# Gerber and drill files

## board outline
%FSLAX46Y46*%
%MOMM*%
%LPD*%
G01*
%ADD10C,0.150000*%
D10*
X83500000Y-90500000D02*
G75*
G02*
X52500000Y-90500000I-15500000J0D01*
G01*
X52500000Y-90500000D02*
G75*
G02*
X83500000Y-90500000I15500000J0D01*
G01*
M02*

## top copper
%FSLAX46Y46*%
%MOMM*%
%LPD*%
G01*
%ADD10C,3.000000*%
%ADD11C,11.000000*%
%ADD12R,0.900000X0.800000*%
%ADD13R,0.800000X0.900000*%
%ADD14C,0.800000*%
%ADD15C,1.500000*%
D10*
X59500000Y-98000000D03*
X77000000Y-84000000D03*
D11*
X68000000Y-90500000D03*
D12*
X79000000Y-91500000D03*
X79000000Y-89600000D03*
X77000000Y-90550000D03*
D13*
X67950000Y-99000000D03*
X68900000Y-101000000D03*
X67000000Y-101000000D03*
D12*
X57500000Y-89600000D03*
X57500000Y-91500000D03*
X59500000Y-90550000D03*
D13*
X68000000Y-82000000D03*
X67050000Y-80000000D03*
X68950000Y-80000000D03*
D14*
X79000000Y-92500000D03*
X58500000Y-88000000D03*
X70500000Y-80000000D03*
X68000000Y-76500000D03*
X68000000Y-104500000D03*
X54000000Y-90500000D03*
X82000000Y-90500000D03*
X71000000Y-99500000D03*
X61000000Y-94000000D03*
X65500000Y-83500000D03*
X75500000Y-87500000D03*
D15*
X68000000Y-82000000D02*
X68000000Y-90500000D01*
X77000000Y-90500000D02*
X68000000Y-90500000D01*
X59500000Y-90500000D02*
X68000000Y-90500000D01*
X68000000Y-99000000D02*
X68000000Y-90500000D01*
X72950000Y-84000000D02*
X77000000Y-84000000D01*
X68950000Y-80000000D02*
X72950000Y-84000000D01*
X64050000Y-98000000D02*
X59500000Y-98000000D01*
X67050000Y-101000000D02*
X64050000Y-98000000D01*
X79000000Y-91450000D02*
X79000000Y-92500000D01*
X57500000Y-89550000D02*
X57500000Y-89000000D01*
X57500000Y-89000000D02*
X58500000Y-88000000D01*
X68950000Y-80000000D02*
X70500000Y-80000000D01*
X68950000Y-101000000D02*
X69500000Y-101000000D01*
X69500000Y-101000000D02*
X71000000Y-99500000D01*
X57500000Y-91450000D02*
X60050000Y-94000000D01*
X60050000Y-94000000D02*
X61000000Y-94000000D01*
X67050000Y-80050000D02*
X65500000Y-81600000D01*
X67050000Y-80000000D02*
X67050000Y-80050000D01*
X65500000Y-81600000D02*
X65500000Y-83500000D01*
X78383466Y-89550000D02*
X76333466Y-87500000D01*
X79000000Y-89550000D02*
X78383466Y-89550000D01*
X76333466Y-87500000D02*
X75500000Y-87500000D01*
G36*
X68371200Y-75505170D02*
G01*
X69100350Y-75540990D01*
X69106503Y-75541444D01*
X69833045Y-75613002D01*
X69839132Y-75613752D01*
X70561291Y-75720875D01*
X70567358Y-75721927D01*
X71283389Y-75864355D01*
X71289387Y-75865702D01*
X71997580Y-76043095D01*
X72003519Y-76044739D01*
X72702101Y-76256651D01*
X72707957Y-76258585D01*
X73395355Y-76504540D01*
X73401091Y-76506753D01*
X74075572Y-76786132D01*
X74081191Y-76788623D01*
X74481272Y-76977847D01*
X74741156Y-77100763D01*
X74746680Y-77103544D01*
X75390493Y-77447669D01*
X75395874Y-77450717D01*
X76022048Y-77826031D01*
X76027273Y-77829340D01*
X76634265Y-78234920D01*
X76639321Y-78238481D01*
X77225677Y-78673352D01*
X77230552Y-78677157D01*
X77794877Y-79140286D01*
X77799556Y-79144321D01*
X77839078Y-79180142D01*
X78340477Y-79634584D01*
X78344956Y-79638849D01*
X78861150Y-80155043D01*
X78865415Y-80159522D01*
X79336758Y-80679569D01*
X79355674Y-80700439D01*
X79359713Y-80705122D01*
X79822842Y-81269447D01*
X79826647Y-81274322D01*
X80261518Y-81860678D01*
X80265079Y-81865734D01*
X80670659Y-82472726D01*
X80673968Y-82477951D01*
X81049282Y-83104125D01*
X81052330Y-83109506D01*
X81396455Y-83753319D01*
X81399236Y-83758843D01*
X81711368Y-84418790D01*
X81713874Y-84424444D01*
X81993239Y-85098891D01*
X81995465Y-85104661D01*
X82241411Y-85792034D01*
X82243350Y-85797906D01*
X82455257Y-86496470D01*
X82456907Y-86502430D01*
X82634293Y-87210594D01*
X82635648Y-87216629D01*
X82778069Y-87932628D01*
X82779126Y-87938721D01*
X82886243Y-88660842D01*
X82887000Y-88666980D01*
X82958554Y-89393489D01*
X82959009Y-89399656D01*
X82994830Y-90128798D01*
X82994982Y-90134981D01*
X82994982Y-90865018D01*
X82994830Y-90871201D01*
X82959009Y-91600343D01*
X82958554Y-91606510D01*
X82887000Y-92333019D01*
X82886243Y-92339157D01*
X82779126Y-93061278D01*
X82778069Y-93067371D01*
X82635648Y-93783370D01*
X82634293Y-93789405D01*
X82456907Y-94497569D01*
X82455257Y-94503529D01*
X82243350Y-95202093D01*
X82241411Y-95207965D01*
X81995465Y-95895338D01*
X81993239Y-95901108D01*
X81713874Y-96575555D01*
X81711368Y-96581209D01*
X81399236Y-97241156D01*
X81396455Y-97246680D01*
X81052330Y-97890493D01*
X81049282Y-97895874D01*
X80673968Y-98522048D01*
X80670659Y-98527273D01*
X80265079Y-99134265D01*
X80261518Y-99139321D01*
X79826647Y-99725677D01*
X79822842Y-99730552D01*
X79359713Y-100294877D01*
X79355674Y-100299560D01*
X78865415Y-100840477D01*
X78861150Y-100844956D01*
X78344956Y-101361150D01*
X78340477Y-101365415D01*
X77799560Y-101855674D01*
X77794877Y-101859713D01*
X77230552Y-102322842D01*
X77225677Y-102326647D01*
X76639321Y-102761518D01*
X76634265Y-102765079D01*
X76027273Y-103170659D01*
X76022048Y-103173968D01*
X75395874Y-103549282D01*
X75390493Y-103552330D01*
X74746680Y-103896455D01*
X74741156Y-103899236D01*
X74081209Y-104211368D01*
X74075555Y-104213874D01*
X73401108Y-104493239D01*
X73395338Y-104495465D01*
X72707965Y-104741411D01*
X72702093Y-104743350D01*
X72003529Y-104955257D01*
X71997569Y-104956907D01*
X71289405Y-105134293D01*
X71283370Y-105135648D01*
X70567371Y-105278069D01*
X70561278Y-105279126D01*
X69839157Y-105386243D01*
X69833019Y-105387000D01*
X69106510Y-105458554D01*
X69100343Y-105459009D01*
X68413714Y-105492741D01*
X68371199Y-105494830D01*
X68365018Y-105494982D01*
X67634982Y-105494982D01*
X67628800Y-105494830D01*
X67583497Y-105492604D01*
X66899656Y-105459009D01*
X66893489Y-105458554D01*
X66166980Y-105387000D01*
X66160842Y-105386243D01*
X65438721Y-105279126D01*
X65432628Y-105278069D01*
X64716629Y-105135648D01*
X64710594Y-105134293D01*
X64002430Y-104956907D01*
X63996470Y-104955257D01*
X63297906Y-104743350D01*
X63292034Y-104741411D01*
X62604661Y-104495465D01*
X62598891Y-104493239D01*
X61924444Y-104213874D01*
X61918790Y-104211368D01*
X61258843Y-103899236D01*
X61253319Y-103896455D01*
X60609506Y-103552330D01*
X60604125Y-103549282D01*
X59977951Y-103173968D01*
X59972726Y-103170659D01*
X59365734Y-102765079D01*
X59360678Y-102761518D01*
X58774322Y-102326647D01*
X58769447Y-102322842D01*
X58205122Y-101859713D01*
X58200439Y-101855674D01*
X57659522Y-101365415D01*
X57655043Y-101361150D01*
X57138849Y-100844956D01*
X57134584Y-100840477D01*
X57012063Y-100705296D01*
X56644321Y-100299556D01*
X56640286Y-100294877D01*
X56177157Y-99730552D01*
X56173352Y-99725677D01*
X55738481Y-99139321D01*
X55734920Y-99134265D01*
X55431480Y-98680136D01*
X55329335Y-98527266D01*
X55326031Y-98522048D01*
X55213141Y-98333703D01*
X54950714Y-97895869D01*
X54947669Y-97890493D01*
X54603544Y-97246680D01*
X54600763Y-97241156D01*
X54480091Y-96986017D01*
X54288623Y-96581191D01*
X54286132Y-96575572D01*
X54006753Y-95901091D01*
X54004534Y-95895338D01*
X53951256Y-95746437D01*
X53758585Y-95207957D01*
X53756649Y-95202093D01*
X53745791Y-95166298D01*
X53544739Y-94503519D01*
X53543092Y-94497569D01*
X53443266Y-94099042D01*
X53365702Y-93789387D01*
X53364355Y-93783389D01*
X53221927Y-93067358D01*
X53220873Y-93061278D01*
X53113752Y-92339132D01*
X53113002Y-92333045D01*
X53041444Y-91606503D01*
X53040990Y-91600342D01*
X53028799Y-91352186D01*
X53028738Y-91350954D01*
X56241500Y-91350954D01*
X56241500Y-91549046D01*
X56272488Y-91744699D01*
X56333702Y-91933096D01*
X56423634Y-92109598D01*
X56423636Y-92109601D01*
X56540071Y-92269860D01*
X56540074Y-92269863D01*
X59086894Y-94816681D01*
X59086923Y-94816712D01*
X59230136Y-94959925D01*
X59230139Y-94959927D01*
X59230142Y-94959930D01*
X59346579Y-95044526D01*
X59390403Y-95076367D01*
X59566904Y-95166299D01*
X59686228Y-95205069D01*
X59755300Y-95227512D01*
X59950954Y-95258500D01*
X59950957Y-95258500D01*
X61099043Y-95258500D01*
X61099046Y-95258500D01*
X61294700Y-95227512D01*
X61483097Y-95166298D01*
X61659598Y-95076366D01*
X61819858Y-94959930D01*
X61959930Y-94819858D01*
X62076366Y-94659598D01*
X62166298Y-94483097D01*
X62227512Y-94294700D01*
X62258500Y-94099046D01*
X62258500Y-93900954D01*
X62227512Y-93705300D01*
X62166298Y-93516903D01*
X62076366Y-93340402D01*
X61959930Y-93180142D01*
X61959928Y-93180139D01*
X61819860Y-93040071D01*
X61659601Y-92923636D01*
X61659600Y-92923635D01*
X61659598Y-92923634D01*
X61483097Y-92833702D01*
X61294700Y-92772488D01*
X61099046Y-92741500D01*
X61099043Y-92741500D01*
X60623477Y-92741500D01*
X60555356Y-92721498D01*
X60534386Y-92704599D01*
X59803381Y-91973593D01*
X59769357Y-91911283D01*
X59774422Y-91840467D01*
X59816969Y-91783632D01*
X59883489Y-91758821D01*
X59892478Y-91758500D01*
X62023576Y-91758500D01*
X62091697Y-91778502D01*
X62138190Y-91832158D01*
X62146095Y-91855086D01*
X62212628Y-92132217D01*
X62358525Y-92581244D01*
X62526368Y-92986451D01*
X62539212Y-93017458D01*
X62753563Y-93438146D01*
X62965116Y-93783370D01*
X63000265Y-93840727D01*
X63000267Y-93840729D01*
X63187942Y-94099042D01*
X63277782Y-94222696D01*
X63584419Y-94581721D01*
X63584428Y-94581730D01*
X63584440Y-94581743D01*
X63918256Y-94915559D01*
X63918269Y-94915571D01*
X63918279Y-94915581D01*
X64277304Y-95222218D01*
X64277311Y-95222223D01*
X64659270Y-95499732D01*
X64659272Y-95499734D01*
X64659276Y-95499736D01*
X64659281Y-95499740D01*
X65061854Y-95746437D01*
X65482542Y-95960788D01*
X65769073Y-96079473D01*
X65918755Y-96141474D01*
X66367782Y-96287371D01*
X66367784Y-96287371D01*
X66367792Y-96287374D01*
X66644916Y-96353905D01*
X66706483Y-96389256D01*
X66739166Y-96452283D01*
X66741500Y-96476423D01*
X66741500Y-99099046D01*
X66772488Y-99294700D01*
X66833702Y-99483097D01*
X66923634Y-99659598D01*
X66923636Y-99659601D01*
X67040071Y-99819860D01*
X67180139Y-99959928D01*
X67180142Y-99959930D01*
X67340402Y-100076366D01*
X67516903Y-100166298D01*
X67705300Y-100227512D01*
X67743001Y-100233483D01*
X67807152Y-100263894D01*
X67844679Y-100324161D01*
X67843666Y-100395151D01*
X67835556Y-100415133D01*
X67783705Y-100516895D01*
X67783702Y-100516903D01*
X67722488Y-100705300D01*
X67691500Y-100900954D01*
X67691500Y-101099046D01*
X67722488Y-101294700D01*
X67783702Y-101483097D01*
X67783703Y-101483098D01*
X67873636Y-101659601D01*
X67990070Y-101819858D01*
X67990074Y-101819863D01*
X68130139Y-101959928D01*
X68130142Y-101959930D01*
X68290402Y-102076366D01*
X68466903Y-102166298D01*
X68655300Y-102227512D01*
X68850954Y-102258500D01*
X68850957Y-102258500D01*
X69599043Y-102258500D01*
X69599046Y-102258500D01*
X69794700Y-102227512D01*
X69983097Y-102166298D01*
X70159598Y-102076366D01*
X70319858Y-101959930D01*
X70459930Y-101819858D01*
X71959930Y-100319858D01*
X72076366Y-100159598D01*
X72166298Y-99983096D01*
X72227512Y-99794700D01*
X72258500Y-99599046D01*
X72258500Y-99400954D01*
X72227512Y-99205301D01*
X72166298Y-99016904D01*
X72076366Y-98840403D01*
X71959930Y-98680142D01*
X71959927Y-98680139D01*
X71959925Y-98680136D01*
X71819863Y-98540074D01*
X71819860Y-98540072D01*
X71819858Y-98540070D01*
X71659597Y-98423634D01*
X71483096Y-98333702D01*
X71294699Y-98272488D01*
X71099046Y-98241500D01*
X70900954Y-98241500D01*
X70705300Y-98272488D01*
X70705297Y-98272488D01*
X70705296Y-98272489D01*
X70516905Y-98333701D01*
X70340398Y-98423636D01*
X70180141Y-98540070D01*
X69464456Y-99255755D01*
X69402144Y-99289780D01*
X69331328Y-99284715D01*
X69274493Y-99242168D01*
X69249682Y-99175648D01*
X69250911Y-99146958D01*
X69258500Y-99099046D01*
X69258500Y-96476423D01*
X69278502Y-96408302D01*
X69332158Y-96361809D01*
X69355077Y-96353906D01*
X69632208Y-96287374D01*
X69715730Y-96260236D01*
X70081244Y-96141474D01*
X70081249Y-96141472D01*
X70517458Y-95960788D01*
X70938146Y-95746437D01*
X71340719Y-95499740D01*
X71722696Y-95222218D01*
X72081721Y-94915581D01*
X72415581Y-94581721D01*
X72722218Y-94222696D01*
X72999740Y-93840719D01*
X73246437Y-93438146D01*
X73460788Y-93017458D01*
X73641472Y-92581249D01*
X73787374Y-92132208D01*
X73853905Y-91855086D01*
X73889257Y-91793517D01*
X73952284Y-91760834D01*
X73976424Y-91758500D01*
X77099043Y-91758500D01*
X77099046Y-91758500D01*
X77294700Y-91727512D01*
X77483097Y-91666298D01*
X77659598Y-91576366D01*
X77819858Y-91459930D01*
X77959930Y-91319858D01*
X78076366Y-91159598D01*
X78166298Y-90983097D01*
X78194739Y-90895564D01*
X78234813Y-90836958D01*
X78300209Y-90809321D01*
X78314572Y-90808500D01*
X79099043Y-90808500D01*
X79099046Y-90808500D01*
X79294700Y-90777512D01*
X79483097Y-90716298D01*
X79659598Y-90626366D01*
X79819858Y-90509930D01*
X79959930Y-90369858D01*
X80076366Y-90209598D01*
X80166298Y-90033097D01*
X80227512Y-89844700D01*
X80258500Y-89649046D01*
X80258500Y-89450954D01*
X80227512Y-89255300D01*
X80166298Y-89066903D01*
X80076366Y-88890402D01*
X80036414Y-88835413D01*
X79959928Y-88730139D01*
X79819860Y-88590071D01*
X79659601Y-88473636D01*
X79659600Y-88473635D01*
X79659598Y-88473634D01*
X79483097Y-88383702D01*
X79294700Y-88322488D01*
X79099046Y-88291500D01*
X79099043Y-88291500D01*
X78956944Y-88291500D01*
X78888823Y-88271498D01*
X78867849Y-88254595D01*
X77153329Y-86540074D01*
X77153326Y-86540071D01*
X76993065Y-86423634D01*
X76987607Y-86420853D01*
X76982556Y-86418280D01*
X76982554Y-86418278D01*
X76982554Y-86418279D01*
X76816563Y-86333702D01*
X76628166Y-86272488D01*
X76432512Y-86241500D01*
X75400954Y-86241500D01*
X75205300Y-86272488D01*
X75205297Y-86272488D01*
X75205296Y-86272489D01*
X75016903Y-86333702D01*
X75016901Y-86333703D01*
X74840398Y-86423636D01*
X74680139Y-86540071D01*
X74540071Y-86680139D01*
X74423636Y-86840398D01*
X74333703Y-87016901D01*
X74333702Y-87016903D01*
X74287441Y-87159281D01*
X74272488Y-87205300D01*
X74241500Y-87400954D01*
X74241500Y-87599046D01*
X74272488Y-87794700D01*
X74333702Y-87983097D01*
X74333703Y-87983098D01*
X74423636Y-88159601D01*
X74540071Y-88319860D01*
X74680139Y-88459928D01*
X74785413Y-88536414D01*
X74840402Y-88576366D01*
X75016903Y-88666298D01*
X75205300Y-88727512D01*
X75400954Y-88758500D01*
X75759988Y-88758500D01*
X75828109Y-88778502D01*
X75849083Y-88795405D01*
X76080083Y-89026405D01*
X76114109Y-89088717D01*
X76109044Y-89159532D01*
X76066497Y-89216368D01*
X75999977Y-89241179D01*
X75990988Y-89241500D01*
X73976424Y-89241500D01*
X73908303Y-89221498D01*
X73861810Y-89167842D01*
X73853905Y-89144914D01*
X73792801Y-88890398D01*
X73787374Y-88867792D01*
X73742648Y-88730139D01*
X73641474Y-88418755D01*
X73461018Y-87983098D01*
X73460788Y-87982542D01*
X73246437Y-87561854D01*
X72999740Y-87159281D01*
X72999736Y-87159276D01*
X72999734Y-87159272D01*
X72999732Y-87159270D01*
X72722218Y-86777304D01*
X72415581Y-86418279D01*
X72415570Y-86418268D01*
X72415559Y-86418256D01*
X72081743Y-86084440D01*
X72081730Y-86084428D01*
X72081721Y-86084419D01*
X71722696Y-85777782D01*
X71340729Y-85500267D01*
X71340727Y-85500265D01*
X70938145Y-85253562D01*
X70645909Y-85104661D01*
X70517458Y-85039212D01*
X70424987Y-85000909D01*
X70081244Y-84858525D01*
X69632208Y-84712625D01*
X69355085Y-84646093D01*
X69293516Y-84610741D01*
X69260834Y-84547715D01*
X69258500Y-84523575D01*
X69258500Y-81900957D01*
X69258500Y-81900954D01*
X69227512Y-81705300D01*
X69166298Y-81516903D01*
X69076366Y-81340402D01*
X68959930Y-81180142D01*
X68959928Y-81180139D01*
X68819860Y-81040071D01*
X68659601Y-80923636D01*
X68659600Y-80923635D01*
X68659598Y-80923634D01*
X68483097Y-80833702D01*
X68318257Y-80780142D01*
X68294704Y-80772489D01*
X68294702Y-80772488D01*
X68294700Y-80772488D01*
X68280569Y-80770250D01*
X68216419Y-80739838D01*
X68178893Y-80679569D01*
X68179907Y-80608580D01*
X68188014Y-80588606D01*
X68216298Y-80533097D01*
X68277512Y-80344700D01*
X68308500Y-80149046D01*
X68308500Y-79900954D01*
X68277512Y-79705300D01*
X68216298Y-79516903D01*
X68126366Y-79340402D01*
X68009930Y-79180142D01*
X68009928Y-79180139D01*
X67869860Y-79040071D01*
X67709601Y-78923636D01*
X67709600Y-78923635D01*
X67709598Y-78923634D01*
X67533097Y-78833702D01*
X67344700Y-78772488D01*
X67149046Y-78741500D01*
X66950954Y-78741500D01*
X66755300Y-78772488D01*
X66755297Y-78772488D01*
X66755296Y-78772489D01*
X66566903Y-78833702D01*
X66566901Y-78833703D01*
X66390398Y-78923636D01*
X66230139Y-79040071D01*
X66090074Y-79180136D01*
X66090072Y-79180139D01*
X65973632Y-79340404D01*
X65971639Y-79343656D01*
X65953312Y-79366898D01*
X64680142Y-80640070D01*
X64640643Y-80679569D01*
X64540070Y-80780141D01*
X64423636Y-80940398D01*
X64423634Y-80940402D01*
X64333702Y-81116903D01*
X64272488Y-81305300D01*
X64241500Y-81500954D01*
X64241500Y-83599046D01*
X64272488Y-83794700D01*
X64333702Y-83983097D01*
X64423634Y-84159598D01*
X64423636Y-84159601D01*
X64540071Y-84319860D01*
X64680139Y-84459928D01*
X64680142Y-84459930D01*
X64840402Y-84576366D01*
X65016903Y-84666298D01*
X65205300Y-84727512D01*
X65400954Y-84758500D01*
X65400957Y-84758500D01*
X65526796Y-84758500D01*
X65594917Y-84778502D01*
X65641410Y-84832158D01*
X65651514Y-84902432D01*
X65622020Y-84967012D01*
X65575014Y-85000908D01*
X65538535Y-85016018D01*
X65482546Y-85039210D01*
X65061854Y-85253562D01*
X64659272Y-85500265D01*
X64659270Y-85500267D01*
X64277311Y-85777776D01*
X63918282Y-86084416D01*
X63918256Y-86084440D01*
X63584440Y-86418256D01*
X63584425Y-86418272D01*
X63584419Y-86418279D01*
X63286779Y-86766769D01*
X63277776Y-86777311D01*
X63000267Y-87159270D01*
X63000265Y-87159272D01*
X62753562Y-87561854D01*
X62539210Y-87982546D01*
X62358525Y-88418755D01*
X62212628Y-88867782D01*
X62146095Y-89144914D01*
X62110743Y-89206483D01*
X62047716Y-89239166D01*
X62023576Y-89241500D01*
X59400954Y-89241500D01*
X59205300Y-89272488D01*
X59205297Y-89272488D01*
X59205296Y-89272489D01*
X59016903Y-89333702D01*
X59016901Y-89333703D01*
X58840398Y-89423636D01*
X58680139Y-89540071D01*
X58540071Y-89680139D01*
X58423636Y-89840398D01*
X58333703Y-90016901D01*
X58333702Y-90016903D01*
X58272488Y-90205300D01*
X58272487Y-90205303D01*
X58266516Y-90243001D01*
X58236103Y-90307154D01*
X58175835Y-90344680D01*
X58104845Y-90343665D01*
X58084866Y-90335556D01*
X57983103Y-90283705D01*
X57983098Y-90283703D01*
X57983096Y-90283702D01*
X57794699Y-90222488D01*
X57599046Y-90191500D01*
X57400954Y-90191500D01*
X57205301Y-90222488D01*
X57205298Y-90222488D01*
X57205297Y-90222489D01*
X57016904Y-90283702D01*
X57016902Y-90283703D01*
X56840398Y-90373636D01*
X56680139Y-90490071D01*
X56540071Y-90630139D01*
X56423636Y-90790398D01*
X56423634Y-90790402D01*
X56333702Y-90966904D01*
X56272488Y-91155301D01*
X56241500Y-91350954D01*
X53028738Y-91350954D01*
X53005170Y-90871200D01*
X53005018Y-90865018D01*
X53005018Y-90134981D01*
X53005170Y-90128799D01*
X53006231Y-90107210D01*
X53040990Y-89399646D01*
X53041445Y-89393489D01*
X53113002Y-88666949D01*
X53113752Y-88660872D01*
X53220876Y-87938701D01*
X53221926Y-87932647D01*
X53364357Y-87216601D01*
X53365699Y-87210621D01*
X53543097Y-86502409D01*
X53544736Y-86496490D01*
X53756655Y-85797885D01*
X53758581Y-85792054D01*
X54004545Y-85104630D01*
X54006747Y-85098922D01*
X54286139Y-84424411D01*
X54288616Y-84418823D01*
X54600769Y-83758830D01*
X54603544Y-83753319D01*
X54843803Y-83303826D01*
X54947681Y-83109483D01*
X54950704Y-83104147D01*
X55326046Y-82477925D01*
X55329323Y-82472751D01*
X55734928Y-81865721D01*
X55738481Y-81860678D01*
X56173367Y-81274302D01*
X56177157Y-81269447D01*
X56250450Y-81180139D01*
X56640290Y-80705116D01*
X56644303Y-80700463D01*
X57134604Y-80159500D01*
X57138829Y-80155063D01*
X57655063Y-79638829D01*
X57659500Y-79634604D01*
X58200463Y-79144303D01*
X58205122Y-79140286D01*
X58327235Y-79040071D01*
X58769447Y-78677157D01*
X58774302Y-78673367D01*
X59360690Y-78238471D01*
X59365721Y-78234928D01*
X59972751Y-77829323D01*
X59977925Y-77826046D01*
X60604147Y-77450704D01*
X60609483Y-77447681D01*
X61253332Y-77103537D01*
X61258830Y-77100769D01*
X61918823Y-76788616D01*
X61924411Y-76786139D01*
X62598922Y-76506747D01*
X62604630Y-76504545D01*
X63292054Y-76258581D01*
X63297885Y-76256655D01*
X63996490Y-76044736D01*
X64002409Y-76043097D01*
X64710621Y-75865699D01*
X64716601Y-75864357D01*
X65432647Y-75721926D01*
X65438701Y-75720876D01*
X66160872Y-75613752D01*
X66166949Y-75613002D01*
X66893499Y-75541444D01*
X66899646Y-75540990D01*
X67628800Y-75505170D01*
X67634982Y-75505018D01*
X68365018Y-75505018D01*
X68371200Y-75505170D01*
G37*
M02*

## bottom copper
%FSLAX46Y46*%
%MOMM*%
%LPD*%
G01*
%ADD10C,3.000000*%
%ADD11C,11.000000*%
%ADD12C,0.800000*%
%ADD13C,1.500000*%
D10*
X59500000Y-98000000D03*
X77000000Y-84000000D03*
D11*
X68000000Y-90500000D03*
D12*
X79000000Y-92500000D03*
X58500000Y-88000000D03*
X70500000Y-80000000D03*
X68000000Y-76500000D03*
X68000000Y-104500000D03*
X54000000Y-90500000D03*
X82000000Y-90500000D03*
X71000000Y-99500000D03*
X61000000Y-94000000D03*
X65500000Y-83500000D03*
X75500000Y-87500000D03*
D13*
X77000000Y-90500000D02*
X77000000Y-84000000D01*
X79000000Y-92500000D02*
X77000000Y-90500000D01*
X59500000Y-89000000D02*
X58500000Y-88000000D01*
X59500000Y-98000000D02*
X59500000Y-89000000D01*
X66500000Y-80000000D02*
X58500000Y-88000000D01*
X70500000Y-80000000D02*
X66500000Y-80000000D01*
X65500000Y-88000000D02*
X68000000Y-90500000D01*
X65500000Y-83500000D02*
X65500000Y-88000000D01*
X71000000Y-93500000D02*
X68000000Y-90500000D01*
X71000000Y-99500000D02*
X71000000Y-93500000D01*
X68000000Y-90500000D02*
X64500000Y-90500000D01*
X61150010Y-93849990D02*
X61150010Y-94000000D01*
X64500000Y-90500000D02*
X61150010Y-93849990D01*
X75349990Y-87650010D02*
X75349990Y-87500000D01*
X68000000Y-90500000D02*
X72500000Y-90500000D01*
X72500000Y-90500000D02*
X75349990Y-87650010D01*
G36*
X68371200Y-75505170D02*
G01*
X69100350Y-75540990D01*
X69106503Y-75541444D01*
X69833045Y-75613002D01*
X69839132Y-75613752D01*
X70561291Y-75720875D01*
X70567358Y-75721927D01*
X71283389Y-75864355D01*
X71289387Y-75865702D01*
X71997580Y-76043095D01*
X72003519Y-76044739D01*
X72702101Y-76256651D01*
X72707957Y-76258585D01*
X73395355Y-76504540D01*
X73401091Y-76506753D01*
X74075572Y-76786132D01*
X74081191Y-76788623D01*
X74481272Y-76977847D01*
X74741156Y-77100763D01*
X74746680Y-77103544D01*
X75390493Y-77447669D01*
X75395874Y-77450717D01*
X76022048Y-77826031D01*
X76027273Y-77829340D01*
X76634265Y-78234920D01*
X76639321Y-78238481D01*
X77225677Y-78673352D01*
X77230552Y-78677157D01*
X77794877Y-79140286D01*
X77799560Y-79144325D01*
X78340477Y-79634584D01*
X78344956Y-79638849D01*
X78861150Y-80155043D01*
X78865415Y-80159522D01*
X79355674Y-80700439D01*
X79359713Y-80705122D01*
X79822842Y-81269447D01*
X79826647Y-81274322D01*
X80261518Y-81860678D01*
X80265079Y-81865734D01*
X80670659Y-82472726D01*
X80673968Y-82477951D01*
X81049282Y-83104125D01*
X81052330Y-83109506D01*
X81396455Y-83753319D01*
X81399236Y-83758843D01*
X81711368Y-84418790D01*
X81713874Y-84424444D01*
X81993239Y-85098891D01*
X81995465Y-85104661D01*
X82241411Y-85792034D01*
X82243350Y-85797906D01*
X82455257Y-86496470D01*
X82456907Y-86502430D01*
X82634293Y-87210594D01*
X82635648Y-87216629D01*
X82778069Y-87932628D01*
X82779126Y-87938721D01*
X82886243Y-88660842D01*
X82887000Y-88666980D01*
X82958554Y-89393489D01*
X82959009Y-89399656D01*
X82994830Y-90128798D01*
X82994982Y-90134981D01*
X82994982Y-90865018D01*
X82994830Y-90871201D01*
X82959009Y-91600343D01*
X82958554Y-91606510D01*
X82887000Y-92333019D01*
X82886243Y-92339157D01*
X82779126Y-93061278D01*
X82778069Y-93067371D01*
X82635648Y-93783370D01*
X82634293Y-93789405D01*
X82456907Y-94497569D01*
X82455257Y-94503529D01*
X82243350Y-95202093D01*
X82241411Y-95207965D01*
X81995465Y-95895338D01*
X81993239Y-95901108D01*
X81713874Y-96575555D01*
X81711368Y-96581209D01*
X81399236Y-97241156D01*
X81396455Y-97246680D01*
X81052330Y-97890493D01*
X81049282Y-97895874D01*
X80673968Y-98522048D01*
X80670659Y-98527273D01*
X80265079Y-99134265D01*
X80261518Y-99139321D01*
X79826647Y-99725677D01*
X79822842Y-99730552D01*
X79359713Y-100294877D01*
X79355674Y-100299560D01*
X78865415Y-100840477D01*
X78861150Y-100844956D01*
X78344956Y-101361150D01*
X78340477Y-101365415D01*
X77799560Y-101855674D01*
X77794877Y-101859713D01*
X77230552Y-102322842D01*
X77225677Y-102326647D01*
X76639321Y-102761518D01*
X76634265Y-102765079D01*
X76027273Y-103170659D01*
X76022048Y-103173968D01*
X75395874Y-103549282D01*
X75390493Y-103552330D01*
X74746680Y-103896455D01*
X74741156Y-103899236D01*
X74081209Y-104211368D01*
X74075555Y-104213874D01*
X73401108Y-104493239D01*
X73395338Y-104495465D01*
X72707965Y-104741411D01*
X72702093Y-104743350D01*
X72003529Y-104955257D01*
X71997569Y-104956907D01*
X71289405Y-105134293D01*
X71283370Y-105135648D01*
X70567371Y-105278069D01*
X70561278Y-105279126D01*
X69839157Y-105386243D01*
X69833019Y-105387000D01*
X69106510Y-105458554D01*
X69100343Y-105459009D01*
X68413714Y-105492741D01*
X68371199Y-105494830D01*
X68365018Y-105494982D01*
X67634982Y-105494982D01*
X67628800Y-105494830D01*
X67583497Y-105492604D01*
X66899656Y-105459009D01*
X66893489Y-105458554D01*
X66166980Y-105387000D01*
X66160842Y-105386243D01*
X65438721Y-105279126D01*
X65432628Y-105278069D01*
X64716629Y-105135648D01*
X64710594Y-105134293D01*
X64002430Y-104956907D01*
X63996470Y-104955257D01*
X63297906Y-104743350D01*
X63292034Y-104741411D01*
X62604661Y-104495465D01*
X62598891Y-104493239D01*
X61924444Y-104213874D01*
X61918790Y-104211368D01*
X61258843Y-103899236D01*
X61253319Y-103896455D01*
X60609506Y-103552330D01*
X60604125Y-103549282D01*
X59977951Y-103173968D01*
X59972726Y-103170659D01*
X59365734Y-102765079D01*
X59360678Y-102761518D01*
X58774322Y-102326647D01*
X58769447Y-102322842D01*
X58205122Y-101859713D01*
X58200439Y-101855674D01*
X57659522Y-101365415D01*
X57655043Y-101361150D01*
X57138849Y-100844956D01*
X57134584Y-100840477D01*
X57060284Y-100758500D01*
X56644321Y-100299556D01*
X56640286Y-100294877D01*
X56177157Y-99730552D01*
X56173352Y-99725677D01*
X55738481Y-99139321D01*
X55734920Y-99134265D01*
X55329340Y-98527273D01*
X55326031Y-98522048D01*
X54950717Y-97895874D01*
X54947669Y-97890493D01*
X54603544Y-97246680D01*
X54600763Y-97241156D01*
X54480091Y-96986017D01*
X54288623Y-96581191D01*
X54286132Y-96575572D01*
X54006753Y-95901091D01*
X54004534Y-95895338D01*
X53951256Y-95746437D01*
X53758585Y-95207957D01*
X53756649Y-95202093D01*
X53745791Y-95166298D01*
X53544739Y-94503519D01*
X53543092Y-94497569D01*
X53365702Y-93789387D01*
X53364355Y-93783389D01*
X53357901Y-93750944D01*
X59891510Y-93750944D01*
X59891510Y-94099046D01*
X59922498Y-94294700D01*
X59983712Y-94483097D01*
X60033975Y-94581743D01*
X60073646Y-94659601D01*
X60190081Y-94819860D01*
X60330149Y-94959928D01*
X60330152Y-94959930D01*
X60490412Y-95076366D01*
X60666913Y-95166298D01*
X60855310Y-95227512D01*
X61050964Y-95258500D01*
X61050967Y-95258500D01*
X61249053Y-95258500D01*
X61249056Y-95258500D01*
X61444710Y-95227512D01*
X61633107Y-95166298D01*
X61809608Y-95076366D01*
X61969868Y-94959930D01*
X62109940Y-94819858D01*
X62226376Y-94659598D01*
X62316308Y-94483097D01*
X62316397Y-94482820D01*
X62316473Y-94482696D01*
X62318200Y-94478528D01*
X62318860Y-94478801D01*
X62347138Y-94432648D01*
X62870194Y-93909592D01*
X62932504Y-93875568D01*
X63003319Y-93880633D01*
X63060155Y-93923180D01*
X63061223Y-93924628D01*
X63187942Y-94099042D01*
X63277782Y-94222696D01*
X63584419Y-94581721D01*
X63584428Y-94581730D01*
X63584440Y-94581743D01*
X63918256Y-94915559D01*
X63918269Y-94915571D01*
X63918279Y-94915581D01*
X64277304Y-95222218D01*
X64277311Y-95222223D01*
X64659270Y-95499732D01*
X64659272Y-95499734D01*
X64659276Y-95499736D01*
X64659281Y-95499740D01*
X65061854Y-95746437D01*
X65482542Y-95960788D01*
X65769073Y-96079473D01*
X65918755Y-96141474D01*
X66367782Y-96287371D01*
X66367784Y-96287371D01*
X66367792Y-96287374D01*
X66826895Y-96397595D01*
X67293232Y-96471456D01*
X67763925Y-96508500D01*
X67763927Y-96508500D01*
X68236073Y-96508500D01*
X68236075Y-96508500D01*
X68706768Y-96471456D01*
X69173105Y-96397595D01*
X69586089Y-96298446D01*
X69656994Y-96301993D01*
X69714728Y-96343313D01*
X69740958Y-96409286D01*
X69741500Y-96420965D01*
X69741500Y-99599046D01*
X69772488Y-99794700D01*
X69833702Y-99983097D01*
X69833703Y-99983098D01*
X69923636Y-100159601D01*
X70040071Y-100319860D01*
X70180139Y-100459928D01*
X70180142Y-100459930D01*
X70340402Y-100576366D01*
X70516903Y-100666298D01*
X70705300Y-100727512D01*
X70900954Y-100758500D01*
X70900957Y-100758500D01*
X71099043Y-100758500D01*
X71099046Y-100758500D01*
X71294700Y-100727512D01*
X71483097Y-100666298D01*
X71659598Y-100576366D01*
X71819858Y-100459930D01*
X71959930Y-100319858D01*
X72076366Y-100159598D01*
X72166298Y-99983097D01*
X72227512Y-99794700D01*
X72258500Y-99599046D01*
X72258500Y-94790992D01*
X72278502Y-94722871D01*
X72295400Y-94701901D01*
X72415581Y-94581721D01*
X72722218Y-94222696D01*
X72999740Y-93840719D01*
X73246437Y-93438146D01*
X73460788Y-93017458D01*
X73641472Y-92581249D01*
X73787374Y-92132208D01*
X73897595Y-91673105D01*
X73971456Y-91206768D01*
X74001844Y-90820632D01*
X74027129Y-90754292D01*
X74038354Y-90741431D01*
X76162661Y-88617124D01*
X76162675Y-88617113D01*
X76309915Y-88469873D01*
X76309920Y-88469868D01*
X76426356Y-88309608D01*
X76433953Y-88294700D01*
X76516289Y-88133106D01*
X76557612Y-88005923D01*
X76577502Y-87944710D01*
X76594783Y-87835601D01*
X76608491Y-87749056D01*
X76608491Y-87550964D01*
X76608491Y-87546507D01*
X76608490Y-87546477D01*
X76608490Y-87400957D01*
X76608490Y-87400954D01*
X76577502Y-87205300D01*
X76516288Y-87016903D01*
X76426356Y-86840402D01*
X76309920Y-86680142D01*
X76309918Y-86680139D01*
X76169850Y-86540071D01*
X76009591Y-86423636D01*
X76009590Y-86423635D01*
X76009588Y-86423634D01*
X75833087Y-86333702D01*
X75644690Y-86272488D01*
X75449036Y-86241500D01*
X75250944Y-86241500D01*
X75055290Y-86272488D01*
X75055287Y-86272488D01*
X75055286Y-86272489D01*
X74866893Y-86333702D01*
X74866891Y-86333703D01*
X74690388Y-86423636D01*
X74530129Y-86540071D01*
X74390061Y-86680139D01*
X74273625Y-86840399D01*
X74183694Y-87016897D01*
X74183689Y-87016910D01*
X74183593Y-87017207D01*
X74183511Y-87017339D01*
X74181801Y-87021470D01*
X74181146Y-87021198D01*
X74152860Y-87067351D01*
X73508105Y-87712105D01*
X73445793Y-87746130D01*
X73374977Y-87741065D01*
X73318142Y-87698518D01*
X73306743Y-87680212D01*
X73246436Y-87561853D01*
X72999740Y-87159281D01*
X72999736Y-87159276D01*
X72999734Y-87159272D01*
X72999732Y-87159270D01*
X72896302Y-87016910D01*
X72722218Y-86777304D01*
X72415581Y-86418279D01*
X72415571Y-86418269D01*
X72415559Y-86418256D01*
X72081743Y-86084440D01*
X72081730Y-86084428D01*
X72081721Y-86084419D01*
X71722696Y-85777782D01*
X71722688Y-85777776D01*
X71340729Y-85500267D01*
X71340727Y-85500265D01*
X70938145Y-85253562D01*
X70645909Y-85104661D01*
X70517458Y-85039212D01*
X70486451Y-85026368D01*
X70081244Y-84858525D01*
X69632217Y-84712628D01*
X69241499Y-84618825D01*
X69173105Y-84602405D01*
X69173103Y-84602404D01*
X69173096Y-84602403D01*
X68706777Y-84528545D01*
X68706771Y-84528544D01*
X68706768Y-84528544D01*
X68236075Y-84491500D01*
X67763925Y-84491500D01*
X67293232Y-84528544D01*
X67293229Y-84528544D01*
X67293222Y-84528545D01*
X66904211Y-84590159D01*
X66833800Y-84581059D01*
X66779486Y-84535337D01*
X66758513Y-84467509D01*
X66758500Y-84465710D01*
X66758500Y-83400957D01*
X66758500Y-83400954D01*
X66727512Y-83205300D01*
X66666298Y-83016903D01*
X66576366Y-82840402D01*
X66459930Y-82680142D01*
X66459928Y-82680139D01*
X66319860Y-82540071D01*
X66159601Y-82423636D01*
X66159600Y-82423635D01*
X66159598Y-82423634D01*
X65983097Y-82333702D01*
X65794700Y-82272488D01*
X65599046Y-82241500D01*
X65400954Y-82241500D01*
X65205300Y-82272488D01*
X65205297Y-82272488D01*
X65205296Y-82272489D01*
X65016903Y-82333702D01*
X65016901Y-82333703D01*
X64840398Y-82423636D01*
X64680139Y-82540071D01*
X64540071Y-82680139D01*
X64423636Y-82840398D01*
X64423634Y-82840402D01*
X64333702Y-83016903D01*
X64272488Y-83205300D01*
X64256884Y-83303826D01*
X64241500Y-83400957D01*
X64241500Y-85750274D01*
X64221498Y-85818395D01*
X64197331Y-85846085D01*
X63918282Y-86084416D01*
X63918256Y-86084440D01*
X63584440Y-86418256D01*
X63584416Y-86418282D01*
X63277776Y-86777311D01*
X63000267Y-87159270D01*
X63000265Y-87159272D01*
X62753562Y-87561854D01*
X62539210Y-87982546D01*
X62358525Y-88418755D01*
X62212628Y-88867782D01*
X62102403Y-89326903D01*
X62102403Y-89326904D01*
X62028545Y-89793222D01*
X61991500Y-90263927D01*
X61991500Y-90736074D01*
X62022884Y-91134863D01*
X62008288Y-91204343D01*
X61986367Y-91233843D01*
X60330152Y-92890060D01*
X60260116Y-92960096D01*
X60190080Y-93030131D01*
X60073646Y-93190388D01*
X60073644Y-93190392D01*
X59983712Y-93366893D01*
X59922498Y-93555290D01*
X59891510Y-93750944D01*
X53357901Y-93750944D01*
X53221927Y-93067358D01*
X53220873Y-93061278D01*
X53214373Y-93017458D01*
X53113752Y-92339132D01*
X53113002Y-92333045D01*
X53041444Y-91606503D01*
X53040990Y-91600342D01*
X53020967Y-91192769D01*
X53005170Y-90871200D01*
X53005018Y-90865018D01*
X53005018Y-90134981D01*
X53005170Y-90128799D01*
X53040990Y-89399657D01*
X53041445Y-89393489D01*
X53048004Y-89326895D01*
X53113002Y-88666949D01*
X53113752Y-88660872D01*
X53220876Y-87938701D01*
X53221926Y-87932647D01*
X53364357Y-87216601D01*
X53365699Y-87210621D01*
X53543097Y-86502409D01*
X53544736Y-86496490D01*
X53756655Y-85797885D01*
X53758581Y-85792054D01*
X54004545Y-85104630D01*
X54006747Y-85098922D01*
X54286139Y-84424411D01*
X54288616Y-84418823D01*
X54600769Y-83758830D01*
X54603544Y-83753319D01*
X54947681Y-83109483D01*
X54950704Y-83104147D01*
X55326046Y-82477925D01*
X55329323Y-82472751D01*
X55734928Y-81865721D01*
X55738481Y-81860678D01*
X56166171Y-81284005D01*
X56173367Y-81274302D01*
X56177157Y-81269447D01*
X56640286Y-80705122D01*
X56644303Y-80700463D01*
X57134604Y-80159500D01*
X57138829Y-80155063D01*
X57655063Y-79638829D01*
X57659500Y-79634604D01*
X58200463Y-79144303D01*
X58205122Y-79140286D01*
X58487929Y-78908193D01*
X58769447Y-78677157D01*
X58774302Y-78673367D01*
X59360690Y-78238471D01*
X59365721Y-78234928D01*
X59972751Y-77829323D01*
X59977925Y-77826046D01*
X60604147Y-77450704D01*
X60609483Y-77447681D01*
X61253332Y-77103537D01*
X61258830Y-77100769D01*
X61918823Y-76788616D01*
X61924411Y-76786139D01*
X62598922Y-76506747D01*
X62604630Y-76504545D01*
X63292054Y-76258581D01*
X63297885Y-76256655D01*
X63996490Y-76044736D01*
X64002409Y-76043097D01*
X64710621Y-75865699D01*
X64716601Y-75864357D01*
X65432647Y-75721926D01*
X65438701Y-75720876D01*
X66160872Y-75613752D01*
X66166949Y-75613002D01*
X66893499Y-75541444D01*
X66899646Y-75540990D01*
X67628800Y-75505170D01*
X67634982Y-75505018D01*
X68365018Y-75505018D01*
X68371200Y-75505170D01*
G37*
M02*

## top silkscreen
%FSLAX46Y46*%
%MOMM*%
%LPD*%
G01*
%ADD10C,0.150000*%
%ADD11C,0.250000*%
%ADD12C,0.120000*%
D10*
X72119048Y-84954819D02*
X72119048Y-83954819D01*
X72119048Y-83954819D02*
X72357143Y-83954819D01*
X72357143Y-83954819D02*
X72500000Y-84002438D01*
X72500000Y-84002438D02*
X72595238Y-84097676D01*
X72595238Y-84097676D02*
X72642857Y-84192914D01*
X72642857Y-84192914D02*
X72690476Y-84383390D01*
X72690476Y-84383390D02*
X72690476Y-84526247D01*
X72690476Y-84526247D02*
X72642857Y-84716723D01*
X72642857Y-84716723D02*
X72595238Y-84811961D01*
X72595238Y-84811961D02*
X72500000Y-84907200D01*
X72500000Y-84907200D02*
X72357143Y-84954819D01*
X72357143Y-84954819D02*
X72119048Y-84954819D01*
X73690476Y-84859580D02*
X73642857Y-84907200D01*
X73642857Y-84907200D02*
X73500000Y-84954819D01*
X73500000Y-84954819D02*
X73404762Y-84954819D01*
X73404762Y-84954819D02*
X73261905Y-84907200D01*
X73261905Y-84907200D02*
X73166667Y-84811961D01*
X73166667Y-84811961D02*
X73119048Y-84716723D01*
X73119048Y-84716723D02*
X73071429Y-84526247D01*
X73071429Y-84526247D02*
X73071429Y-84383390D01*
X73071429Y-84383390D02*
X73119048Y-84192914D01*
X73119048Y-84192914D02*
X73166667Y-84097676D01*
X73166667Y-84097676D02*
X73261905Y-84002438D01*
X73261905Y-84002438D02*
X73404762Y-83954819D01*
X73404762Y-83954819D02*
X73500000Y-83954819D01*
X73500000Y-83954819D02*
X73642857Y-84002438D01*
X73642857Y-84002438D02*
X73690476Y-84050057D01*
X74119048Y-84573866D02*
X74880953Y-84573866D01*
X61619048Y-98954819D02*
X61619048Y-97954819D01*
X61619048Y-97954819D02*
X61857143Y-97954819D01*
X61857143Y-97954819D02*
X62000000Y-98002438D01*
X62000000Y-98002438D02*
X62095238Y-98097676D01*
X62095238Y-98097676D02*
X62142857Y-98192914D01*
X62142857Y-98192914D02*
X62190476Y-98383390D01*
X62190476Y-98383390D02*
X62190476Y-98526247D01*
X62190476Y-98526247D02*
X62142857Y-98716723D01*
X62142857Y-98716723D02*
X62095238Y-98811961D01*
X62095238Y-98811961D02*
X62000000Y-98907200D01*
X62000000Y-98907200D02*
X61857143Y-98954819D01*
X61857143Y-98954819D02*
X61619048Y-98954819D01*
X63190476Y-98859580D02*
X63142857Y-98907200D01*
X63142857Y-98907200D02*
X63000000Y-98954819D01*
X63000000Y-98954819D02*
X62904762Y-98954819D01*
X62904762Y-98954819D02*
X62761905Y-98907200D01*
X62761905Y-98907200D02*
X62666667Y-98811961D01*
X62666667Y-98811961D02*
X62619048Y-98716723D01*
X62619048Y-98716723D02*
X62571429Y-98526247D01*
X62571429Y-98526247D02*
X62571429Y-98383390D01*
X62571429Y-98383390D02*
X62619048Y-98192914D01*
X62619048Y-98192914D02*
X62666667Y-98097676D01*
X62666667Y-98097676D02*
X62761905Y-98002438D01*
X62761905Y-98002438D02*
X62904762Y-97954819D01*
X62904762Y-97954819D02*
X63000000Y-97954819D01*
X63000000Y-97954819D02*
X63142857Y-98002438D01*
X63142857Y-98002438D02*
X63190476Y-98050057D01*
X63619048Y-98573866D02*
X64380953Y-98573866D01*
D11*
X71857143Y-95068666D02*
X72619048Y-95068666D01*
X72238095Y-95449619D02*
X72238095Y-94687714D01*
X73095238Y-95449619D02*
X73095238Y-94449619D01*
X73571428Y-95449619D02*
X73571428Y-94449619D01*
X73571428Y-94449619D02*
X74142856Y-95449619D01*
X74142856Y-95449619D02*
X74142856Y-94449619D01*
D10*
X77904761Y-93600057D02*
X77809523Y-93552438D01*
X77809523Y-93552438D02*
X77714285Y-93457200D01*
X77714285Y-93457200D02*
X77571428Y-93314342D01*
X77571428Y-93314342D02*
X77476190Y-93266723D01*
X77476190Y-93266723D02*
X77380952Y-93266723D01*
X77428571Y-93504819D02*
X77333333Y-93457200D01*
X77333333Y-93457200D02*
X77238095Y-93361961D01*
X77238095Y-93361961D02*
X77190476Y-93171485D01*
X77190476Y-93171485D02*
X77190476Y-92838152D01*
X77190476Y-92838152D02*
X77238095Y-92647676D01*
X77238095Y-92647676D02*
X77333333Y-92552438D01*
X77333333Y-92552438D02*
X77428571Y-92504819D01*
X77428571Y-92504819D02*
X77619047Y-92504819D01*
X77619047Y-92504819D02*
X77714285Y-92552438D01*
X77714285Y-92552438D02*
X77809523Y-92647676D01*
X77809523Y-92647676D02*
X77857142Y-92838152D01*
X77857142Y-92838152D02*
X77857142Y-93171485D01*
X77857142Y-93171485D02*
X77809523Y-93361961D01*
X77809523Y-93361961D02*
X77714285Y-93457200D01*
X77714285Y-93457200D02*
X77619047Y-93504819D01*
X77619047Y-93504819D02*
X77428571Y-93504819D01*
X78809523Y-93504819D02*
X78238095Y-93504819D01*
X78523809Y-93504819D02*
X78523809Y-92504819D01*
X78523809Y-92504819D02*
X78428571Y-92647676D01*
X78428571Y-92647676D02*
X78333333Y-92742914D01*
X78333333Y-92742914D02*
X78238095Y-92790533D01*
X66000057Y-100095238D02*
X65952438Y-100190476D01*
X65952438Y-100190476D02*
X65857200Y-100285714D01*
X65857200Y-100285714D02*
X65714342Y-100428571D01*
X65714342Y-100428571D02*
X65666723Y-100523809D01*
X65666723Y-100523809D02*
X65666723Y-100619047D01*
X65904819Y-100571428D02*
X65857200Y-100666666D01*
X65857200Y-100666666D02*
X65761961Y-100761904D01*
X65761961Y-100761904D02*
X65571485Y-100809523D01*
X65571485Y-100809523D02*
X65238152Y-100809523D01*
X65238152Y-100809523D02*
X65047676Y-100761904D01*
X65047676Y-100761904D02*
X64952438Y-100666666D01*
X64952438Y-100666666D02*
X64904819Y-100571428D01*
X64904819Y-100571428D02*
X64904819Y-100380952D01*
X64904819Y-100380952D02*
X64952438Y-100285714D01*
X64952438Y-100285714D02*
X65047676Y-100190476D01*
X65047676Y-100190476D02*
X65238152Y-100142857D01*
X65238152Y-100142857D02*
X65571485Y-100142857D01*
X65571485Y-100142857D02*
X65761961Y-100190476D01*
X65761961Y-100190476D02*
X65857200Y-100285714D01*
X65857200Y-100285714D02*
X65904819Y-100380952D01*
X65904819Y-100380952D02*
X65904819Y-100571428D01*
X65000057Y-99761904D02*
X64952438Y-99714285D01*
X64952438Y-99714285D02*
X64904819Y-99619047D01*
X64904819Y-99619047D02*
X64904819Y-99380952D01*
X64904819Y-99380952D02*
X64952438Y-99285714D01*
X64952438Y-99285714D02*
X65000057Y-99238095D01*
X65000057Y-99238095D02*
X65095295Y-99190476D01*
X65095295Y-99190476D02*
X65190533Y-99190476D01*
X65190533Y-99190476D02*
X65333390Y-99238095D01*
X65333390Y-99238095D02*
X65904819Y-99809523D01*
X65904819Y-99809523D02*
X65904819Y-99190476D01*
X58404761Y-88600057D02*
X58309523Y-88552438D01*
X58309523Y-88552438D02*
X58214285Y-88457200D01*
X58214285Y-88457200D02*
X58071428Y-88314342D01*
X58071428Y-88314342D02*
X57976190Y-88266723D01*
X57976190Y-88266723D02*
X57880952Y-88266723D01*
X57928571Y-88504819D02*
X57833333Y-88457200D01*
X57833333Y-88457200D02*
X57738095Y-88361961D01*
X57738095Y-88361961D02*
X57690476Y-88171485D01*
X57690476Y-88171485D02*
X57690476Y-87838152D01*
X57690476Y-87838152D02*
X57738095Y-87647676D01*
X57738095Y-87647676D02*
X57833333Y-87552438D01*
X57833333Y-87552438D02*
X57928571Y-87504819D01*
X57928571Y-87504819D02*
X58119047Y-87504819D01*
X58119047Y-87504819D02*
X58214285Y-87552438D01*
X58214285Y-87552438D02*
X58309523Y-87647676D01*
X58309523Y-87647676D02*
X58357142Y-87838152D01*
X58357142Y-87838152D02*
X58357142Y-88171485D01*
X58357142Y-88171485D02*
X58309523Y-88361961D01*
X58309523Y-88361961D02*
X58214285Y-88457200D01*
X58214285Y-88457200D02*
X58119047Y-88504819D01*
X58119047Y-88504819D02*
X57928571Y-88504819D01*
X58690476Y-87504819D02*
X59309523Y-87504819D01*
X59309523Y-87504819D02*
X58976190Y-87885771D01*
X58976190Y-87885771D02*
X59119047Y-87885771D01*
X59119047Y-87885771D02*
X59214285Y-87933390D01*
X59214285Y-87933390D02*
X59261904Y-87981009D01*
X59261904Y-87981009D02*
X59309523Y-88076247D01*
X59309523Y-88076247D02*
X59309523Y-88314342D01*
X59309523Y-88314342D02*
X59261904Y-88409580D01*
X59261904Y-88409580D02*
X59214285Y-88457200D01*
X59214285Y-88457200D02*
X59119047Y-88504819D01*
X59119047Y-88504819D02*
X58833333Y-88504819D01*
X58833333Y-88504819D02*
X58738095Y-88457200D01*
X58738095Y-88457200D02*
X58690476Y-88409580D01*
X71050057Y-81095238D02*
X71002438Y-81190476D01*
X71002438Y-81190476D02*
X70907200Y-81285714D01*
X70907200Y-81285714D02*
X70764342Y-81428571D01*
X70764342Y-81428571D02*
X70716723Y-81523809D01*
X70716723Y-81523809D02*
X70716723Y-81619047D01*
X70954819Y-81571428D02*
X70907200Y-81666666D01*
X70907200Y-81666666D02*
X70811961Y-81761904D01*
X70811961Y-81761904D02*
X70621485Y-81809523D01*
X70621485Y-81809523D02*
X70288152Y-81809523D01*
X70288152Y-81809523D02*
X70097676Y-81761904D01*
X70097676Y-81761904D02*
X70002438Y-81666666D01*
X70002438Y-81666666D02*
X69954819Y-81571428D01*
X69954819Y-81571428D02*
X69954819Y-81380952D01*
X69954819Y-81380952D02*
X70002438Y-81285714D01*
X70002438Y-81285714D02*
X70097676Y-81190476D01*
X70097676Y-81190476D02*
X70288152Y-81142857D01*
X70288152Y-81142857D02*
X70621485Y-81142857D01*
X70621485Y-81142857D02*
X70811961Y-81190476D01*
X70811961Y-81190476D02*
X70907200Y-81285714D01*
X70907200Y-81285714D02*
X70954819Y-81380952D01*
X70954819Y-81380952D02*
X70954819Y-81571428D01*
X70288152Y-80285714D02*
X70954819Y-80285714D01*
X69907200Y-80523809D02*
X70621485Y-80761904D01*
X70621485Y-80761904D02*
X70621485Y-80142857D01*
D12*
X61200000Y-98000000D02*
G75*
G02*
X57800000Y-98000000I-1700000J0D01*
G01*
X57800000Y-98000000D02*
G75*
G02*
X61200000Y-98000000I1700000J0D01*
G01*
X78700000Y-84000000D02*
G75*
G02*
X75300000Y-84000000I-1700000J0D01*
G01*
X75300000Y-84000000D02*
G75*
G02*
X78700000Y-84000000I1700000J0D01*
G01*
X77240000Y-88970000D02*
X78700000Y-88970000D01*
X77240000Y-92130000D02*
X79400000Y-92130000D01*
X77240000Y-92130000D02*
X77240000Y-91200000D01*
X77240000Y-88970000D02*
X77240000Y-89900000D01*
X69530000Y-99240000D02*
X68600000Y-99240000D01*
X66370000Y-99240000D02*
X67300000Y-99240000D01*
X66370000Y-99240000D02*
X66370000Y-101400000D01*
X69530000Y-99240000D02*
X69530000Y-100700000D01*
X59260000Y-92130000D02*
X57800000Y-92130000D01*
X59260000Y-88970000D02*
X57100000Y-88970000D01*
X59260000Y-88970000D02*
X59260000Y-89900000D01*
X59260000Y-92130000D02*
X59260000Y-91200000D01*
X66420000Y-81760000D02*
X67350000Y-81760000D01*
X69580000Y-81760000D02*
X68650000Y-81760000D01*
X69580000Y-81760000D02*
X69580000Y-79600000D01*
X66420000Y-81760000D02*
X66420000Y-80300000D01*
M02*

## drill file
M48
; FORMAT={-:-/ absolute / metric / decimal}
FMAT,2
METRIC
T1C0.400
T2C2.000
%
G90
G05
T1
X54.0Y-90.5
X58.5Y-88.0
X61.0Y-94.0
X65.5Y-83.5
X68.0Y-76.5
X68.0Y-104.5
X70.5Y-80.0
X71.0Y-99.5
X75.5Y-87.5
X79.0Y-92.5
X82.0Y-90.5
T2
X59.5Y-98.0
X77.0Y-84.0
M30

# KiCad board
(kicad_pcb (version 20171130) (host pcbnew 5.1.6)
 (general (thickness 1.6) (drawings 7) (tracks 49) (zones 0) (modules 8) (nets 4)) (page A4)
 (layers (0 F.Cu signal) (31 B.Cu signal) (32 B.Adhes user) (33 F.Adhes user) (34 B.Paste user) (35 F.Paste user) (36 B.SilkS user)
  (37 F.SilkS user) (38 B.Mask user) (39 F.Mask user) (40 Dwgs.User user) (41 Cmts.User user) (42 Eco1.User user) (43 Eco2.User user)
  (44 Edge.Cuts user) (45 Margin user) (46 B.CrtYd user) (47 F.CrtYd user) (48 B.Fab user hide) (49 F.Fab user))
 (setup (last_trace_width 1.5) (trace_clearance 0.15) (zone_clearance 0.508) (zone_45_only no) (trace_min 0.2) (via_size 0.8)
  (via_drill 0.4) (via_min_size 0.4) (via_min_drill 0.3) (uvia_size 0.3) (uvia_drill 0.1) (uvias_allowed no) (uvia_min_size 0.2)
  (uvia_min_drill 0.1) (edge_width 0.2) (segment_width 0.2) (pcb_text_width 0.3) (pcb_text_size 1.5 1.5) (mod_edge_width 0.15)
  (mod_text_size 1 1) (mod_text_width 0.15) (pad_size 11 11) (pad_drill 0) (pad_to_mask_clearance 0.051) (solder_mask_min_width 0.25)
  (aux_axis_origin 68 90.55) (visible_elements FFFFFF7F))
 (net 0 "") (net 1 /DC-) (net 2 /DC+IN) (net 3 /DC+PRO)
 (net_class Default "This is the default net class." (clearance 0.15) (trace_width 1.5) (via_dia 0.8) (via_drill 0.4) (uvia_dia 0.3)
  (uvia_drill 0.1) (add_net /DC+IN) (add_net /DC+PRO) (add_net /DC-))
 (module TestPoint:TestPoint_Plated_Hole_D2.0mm (layer F.Cu) (at 59.5 98)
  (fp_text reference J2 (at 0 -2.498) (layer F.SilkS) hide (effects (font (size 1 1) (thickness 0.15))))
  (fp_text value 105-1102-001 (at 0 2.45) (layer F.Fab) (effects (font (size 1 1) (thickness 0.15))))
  (fp_circle (center 0 0) (end 0 -1.7) (layer F.SilkS) (width 0.12))
  (pad 1 thru_hole circle (at 0 0) (size 3 3) (drill 2) (layers *.Cu *.Mask) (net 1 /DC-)))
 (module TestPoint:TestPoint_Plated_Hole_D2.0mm (layer F.Cu) (at 77 84)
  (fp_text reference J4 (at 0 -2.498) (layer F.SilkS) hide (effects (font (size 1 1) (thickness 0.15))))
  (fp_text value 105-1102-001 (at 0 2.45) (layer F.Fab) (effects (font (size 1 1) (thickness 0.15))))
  (fp_circle (center 0 0) (end 0 -1.7) (layer F.SilkS) (width 0.12))
  (pad 1 thru_hole circle (at 0 0) (size 3 3) (drill 2) (layers *.Cu *.Mask) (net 1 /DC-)))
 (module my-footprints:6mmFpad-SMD (layer F.Cu) (at 68 90.5)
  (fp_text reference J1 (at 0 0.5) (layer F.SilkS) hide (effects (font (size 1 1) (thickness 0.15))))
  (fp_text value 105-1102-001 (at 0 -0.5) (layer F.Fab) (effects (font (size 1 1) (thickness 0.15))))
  (pad 1 smd circle (at 0 0) (size 11 11) (layers F.Cu F.Paste F.Mask) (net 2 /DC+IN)))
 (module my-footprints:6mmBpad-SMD (layer F.Cu) (at 68 90.5)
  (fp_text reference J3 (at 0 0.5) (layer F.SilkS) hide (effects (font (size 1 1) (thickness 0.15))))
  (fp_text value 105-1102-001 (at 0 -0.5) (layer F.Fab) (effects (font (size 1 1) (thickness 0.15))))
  (pad 1 smd circle (at 0 0) (size 11 11) (layers B.Cu B.Paste B.Mask) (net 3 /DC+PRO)))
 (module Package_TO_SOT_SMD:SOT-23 (layer F.Cu) (at 78 90.55 180)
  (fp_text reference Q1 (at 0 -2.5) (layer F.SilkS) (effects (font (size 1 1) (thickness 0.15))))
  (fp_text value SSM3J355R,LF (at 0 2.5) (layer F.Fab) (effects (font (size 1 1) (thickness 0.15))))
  (fp_line (start 0.76 1.58) (end -0.7 1.58) (layer F.SilkS) (width 0.12))
  (fp_line (start 0.76 -1.58) (end -1.4 -1.58) (layer F.SilkS) (width 0.12))
  (fp_line (start 0.76 -1.58) (end 0.76 -0.65) (layer F.SilkS) (width 0.12))
  (fp_line (start 0.76 1.58) (end 0.76 0.65) (layer F.SilkS) (width 0.12))
  (pad 1 smd rect (at -1 -0.95 180) (size 0.9 0.8) (layers F.Cu F.Paste F.Mask) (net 1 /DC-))
  (pad 2 smd rect (at -1 0.95 180) (size 0.9 0.8) (layers F.Cu F.Paste F.Mask) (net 3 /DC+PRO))
  (pad 3 smd rect (at 1 0 180) (size 0.9 0.8) (layers F.Cu F.Paste F.Mask) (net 2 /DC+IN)))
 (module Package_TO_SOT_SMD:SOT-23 (layer F.Cu) (at 67.95 100 90)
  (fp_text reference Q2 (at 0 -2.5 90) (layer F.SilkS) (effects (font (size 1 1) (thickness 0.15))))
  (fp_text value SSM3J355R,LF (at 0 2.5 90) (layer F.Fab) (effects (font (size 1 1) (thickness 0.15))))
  (fp_line (start 0.76 1.58) (end 0.76 0.65) (layer F.SilkS) (width 0.12))
  (fp_line (start 0.76 -1.58) (end 0.76 -0.65) (layer F.SilkS) (width 0.12))
  (fp_line (start 0.76 -1.58) (end -1.4 -1.58) (layer F.SilkS) (width 0.12))
  (fp_line (start 0.76 1.58) (end -0.7 1.58) (layer F.SilkS) (width 0.12))
  (pad 3 smd rect (at 1 0 90) (size 0.9 0.8) (layers F.Cu F.Paste F.Mask) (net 2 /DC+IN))
  (pad 2 smd rect (at -1 0.95 90) (size 0.9 0.8) (layers F.Cu F.Paste F.Mask) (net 3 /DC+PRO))
  (pad 1 smd rect (at -1 -0.95 90) (size 0.9 0.8) (layers F.Cu F.Paste F.Mask) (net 1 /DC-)))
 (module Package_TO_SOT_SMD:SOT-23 (layer F.Cu) (at 58.5 90.55)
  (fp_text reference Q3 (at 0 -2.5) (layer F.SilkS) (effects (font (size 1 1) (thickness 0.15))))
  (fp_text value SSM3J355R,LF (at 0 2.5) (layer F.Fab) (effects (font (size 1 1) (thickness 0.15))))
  (fp_line (start 0.76 1.58) (end -0.7 1.58) (layer F.SilkS) (width 0.12))
  (fp_line (start 0.76 -1.58) (end -1.4 -1.58) (layer F.SilkS) (width 0.12))
  (fp_line (start 0.76 -1.58) (end 0.76 -0.65) (layer F.SilkS) (width 0.12))
  (fp_line (start 0.76 1.58) (end 0.76 0.65) (layer F.SilkS) (width 0.12))
  (pad 1 smd rect (at -1 -0.95) (size 0.9 0.8) (layers F.Cu F.Paste F.Mask) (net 1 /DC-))
  (pad 2 smd rect (at -1 0.95) (size 0.9 0.8) (layers F.Cu F.Paste F.Mask) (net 3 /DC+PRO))
  (pad 3 smd rect (at 1 0) (size 0.9 0.8) (layers F.Cu F.Paste F.Mask) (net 2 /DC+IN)))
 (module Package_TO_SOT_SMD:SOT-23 (layer F.Cu) (at 68 81 270)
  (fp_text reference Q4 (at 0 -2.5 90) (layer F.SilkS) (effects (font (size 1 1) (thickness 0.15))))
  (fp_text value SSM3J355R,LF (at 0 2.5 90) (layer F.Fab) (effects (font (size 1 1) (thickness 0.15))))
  (fp_line (start 0.76 1.58) (end 0.76 0.65) (layer F.SilkS) (width 0.12))
  (fp_line (start 0.76 -1.58) (end 0.76 -0.65) (layer F.SilkS) (width 0.12))
  (fp_line (start 0.76 -1.58) (end -1.4 -1.58) (layer F.SilkS) (width 0.12))
  (fp_line (start 0.76 1.58) (end -0.7 1.58) (layer F.SilkS) (width 0.12))
  (pad 3 smd rect (at 1 0 270) (size 0.9 0.8) (layers F.Cu F.Paste F.Mask) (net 2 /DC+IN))
  (pad 2 smd rect (at -1 0.95 270) (size 0.9 0.8) (layers F.Cu F.Paste F.Mask) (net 3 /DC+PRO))
  (pad 1 smd rect (at -1 -0.95 270) (size 0.9 0.8) (layers F.Cu F.Paste F.Mask) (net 1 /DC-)))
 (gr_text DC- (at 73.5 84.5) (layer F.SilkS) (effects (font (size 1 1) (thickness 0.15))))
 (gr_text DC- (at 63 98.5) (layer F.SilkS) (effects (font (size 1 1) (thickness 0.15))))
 (gr_circle (center 68 90.5) (end 83.5 90.5) (layer Edge.Cuts) (width 0.15))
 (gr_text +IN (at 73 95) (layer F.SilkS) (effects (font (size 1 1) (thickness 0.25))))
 (segment (start 68 82) (end 68 90.5) (width 1.5) (layer F.Cu) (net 2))
 (segment (start 77 90.5) (end 68 90.5) (width 1.5) (layer F.Cu) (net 2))
 (segment (start 59.5 90.5) (end 68 90.5) (width 1.5) (layer F.Cu) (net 2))
 (segment (start 68 99) (end 68 90.5) (width 1.5) (layer F.Cu) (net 2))
 (segment (start 72.95 84) (end 77 84) (width 1.5) (layer F.Cu) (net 1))
 (segment (start 68.95 80) (end 72.95 84) (width 1.5) (layer F.Cu) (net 1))
 (segment (start 64.05 98) (end 59.5 98) (width 1.5) (layer F.Cu) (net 1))
 (segment (start 67.05 101) (end 64.05 98) (width 1.5) (layer F.Cu) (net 1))
 (segment (start 79 91.45) (end 79 92.5) (width 1.5) (layer F.Cu) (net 1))
 (via (at 79 92.5) (size 0.8) (drill 0.4) (layers F.Cu B.Cu) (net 1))
 (segment (start 77 90.5) (end 77 84) (width 1.5) (layer B.Cu) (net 1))
 (segment (start 79 92.5) (end 77 90.5) (width 1.5) (layer B.Cu) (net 1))
 (segment (start 57.5 89.55) (end 57.5 89) (width 1.5) (layer F.Cu) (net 1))
 (via (at 58.5 88) (size 0.8) (drill 0.4) (layers F.Cu B.Cu) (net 1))
 (segment (start 57.5 89) (end 58.5 88) (width 1.5) (layer F.Cu) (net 1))
 (segment (start 59.5 89) (end 58.5 88) (width 1.5) (layer B.Cu) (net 1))
 (segment (start 59.5 98) (end 59.5 89) (width 1.5) (layer B.Cu) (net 1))
 (segment (start 68.95 80) (end 70.5 80) (width 1.5) (layer F.Cu) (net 1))
 (via (at 70.5 80) (size 0.8) (drill 0.4) (layers F.Cu B.Cu) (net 1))
 (segment (start 66.5 80) (end 58.5 88) (width 1.5) (layer B.Cu) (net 1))
 (segment (start 70.5 80) (end 66.5 80) (width 1.5) (layer B.Cu) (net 1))
 (via (at 68 76.5) (size 0.8) (drill 0.4) (layers F.Cu B.Cu) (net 1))
 (via (at 68 104.5) (size 0.8) (drill 0.4) (layers F.Cu B.Cu) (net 1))
 (via (at 54 90.5) (size 0.8) (drill 0.4) (layers F.Cu B.Cu) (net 1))
 (via (at 82 90.5) (size 0.8) (drill 0.4) (layers F.Cu B.Cu) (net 1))
 (via (at 71 99.5) (size 0.8) (drill 0.4) (layers F.Cu B.Cu) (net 3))
 (segment (start 68.95 101) (end 69.5 101) (width 1.5) (layer F.Cu) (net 3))
 (segment (start 69.5 101) (end 71 99.5) (width 1.5) (layer F.Cu) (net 3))
 (segment (start 57.5 91.45) (end 60.05 94) (width 1.5) (layer F.Cu) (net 3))
 (via (at 61 94) (size 0.8) (drill 0.4) (layers F.Cu B.Cu) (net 3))
 (segment (start 60.05 94) (end 61 94) (width 1.5) (layer F.Cu) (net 3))
 (segment (start 67.05 80.05) (end 65.5 81.6) (width 1.5) (layer F.Cu) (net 3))
 (segment (start 67.05 80) (end 67.05 80.05) (width 1.5) (layer F.Cu) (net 3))
 (via (at 65.5 83.5) (size 0.8) (drill 0.4) (layers F.Cu B.Cu) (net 3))
 (segment (start 65.5 81.6) (end 65.5 83.5) (width 1.5) (layer F.Cu) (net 3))
 (segment (start 65.5 88) (end 68 90.5) (width 1.5) (layer B.Cu) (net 3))
 (segment (start 65.5 83.5) (end 65.5 88) (width 1.5) (layer B.Cu) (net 3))
 (segment (start 71 93.5) (end 68 90.5) (width 1.5) (layer B.Cu) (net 3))
 (segment (start 71 99.5) (end 71 93.5) (width 1.5) (layer B.Cu) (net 3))
 (segment (start 68 90.5) (end 64.5 90.5) (width 1.5) (layer B.Cu) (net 3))
 (segment (start 61.15001 93.84999) (end 61.15001 94) (width 1.5) (layer B.Cu) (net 3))
 (segment (start 64.5 90.5) (end 61.15001 93.84999) (width 1.5) (layer B.Cu) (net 3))
 (segment (start 78.383466 89.55) (end 76.333466 87.5) (width 1.5) (layer F.Cu) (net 3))
 (segment (start 79 89.55) (end 78.383466 89.55) (width 1.5) (layer F.Cu) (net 3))
 (via (at 75.5 87.5) (size 0.8) (drill 0.4) (layers F.Cu B.Cu) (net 3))
 (segment (start 76.333466 87.5) (end 75.5 87.5) (width 1.5) (layer F.Cu) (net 3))
 (segment (start 75.34999 87.65001) (end 75.34999 87.5) (width 1.5) (layer B.Cu) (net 3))
 (segment (start 68 90.5) (end 72.5 90.5) (width 1.5) (layer B.Cu) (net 3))
 (segment (start 72.5 90.5) (end 75.34999 87.65001) (width 1.5) (layer B.Cu) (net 3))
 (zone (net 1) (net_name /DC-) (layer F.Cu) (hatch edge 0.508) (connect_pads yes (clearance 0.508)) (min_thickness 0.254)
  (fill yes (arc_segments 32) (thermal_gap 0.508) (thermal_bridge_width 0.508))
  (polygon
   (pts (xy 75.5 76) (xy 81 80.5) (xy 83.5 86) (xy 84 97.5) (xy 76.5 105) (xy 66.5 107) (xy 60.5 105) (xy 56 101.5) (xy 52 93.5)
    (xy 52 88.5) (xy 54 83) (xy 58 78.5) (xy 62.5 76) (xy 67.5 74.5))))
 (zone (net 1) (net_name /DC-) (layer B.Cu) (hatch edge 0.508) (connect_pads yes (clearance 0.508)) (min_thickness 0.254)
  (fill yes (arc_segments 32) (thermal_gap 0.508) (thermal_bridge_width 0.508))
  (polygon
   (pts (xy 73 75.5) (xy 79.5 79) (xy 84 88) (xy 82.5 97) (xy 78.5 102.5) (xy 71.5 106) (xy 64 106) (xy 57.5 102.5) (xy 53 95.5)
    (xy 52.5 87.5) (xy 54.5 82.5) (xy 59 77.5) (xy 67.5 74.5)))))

